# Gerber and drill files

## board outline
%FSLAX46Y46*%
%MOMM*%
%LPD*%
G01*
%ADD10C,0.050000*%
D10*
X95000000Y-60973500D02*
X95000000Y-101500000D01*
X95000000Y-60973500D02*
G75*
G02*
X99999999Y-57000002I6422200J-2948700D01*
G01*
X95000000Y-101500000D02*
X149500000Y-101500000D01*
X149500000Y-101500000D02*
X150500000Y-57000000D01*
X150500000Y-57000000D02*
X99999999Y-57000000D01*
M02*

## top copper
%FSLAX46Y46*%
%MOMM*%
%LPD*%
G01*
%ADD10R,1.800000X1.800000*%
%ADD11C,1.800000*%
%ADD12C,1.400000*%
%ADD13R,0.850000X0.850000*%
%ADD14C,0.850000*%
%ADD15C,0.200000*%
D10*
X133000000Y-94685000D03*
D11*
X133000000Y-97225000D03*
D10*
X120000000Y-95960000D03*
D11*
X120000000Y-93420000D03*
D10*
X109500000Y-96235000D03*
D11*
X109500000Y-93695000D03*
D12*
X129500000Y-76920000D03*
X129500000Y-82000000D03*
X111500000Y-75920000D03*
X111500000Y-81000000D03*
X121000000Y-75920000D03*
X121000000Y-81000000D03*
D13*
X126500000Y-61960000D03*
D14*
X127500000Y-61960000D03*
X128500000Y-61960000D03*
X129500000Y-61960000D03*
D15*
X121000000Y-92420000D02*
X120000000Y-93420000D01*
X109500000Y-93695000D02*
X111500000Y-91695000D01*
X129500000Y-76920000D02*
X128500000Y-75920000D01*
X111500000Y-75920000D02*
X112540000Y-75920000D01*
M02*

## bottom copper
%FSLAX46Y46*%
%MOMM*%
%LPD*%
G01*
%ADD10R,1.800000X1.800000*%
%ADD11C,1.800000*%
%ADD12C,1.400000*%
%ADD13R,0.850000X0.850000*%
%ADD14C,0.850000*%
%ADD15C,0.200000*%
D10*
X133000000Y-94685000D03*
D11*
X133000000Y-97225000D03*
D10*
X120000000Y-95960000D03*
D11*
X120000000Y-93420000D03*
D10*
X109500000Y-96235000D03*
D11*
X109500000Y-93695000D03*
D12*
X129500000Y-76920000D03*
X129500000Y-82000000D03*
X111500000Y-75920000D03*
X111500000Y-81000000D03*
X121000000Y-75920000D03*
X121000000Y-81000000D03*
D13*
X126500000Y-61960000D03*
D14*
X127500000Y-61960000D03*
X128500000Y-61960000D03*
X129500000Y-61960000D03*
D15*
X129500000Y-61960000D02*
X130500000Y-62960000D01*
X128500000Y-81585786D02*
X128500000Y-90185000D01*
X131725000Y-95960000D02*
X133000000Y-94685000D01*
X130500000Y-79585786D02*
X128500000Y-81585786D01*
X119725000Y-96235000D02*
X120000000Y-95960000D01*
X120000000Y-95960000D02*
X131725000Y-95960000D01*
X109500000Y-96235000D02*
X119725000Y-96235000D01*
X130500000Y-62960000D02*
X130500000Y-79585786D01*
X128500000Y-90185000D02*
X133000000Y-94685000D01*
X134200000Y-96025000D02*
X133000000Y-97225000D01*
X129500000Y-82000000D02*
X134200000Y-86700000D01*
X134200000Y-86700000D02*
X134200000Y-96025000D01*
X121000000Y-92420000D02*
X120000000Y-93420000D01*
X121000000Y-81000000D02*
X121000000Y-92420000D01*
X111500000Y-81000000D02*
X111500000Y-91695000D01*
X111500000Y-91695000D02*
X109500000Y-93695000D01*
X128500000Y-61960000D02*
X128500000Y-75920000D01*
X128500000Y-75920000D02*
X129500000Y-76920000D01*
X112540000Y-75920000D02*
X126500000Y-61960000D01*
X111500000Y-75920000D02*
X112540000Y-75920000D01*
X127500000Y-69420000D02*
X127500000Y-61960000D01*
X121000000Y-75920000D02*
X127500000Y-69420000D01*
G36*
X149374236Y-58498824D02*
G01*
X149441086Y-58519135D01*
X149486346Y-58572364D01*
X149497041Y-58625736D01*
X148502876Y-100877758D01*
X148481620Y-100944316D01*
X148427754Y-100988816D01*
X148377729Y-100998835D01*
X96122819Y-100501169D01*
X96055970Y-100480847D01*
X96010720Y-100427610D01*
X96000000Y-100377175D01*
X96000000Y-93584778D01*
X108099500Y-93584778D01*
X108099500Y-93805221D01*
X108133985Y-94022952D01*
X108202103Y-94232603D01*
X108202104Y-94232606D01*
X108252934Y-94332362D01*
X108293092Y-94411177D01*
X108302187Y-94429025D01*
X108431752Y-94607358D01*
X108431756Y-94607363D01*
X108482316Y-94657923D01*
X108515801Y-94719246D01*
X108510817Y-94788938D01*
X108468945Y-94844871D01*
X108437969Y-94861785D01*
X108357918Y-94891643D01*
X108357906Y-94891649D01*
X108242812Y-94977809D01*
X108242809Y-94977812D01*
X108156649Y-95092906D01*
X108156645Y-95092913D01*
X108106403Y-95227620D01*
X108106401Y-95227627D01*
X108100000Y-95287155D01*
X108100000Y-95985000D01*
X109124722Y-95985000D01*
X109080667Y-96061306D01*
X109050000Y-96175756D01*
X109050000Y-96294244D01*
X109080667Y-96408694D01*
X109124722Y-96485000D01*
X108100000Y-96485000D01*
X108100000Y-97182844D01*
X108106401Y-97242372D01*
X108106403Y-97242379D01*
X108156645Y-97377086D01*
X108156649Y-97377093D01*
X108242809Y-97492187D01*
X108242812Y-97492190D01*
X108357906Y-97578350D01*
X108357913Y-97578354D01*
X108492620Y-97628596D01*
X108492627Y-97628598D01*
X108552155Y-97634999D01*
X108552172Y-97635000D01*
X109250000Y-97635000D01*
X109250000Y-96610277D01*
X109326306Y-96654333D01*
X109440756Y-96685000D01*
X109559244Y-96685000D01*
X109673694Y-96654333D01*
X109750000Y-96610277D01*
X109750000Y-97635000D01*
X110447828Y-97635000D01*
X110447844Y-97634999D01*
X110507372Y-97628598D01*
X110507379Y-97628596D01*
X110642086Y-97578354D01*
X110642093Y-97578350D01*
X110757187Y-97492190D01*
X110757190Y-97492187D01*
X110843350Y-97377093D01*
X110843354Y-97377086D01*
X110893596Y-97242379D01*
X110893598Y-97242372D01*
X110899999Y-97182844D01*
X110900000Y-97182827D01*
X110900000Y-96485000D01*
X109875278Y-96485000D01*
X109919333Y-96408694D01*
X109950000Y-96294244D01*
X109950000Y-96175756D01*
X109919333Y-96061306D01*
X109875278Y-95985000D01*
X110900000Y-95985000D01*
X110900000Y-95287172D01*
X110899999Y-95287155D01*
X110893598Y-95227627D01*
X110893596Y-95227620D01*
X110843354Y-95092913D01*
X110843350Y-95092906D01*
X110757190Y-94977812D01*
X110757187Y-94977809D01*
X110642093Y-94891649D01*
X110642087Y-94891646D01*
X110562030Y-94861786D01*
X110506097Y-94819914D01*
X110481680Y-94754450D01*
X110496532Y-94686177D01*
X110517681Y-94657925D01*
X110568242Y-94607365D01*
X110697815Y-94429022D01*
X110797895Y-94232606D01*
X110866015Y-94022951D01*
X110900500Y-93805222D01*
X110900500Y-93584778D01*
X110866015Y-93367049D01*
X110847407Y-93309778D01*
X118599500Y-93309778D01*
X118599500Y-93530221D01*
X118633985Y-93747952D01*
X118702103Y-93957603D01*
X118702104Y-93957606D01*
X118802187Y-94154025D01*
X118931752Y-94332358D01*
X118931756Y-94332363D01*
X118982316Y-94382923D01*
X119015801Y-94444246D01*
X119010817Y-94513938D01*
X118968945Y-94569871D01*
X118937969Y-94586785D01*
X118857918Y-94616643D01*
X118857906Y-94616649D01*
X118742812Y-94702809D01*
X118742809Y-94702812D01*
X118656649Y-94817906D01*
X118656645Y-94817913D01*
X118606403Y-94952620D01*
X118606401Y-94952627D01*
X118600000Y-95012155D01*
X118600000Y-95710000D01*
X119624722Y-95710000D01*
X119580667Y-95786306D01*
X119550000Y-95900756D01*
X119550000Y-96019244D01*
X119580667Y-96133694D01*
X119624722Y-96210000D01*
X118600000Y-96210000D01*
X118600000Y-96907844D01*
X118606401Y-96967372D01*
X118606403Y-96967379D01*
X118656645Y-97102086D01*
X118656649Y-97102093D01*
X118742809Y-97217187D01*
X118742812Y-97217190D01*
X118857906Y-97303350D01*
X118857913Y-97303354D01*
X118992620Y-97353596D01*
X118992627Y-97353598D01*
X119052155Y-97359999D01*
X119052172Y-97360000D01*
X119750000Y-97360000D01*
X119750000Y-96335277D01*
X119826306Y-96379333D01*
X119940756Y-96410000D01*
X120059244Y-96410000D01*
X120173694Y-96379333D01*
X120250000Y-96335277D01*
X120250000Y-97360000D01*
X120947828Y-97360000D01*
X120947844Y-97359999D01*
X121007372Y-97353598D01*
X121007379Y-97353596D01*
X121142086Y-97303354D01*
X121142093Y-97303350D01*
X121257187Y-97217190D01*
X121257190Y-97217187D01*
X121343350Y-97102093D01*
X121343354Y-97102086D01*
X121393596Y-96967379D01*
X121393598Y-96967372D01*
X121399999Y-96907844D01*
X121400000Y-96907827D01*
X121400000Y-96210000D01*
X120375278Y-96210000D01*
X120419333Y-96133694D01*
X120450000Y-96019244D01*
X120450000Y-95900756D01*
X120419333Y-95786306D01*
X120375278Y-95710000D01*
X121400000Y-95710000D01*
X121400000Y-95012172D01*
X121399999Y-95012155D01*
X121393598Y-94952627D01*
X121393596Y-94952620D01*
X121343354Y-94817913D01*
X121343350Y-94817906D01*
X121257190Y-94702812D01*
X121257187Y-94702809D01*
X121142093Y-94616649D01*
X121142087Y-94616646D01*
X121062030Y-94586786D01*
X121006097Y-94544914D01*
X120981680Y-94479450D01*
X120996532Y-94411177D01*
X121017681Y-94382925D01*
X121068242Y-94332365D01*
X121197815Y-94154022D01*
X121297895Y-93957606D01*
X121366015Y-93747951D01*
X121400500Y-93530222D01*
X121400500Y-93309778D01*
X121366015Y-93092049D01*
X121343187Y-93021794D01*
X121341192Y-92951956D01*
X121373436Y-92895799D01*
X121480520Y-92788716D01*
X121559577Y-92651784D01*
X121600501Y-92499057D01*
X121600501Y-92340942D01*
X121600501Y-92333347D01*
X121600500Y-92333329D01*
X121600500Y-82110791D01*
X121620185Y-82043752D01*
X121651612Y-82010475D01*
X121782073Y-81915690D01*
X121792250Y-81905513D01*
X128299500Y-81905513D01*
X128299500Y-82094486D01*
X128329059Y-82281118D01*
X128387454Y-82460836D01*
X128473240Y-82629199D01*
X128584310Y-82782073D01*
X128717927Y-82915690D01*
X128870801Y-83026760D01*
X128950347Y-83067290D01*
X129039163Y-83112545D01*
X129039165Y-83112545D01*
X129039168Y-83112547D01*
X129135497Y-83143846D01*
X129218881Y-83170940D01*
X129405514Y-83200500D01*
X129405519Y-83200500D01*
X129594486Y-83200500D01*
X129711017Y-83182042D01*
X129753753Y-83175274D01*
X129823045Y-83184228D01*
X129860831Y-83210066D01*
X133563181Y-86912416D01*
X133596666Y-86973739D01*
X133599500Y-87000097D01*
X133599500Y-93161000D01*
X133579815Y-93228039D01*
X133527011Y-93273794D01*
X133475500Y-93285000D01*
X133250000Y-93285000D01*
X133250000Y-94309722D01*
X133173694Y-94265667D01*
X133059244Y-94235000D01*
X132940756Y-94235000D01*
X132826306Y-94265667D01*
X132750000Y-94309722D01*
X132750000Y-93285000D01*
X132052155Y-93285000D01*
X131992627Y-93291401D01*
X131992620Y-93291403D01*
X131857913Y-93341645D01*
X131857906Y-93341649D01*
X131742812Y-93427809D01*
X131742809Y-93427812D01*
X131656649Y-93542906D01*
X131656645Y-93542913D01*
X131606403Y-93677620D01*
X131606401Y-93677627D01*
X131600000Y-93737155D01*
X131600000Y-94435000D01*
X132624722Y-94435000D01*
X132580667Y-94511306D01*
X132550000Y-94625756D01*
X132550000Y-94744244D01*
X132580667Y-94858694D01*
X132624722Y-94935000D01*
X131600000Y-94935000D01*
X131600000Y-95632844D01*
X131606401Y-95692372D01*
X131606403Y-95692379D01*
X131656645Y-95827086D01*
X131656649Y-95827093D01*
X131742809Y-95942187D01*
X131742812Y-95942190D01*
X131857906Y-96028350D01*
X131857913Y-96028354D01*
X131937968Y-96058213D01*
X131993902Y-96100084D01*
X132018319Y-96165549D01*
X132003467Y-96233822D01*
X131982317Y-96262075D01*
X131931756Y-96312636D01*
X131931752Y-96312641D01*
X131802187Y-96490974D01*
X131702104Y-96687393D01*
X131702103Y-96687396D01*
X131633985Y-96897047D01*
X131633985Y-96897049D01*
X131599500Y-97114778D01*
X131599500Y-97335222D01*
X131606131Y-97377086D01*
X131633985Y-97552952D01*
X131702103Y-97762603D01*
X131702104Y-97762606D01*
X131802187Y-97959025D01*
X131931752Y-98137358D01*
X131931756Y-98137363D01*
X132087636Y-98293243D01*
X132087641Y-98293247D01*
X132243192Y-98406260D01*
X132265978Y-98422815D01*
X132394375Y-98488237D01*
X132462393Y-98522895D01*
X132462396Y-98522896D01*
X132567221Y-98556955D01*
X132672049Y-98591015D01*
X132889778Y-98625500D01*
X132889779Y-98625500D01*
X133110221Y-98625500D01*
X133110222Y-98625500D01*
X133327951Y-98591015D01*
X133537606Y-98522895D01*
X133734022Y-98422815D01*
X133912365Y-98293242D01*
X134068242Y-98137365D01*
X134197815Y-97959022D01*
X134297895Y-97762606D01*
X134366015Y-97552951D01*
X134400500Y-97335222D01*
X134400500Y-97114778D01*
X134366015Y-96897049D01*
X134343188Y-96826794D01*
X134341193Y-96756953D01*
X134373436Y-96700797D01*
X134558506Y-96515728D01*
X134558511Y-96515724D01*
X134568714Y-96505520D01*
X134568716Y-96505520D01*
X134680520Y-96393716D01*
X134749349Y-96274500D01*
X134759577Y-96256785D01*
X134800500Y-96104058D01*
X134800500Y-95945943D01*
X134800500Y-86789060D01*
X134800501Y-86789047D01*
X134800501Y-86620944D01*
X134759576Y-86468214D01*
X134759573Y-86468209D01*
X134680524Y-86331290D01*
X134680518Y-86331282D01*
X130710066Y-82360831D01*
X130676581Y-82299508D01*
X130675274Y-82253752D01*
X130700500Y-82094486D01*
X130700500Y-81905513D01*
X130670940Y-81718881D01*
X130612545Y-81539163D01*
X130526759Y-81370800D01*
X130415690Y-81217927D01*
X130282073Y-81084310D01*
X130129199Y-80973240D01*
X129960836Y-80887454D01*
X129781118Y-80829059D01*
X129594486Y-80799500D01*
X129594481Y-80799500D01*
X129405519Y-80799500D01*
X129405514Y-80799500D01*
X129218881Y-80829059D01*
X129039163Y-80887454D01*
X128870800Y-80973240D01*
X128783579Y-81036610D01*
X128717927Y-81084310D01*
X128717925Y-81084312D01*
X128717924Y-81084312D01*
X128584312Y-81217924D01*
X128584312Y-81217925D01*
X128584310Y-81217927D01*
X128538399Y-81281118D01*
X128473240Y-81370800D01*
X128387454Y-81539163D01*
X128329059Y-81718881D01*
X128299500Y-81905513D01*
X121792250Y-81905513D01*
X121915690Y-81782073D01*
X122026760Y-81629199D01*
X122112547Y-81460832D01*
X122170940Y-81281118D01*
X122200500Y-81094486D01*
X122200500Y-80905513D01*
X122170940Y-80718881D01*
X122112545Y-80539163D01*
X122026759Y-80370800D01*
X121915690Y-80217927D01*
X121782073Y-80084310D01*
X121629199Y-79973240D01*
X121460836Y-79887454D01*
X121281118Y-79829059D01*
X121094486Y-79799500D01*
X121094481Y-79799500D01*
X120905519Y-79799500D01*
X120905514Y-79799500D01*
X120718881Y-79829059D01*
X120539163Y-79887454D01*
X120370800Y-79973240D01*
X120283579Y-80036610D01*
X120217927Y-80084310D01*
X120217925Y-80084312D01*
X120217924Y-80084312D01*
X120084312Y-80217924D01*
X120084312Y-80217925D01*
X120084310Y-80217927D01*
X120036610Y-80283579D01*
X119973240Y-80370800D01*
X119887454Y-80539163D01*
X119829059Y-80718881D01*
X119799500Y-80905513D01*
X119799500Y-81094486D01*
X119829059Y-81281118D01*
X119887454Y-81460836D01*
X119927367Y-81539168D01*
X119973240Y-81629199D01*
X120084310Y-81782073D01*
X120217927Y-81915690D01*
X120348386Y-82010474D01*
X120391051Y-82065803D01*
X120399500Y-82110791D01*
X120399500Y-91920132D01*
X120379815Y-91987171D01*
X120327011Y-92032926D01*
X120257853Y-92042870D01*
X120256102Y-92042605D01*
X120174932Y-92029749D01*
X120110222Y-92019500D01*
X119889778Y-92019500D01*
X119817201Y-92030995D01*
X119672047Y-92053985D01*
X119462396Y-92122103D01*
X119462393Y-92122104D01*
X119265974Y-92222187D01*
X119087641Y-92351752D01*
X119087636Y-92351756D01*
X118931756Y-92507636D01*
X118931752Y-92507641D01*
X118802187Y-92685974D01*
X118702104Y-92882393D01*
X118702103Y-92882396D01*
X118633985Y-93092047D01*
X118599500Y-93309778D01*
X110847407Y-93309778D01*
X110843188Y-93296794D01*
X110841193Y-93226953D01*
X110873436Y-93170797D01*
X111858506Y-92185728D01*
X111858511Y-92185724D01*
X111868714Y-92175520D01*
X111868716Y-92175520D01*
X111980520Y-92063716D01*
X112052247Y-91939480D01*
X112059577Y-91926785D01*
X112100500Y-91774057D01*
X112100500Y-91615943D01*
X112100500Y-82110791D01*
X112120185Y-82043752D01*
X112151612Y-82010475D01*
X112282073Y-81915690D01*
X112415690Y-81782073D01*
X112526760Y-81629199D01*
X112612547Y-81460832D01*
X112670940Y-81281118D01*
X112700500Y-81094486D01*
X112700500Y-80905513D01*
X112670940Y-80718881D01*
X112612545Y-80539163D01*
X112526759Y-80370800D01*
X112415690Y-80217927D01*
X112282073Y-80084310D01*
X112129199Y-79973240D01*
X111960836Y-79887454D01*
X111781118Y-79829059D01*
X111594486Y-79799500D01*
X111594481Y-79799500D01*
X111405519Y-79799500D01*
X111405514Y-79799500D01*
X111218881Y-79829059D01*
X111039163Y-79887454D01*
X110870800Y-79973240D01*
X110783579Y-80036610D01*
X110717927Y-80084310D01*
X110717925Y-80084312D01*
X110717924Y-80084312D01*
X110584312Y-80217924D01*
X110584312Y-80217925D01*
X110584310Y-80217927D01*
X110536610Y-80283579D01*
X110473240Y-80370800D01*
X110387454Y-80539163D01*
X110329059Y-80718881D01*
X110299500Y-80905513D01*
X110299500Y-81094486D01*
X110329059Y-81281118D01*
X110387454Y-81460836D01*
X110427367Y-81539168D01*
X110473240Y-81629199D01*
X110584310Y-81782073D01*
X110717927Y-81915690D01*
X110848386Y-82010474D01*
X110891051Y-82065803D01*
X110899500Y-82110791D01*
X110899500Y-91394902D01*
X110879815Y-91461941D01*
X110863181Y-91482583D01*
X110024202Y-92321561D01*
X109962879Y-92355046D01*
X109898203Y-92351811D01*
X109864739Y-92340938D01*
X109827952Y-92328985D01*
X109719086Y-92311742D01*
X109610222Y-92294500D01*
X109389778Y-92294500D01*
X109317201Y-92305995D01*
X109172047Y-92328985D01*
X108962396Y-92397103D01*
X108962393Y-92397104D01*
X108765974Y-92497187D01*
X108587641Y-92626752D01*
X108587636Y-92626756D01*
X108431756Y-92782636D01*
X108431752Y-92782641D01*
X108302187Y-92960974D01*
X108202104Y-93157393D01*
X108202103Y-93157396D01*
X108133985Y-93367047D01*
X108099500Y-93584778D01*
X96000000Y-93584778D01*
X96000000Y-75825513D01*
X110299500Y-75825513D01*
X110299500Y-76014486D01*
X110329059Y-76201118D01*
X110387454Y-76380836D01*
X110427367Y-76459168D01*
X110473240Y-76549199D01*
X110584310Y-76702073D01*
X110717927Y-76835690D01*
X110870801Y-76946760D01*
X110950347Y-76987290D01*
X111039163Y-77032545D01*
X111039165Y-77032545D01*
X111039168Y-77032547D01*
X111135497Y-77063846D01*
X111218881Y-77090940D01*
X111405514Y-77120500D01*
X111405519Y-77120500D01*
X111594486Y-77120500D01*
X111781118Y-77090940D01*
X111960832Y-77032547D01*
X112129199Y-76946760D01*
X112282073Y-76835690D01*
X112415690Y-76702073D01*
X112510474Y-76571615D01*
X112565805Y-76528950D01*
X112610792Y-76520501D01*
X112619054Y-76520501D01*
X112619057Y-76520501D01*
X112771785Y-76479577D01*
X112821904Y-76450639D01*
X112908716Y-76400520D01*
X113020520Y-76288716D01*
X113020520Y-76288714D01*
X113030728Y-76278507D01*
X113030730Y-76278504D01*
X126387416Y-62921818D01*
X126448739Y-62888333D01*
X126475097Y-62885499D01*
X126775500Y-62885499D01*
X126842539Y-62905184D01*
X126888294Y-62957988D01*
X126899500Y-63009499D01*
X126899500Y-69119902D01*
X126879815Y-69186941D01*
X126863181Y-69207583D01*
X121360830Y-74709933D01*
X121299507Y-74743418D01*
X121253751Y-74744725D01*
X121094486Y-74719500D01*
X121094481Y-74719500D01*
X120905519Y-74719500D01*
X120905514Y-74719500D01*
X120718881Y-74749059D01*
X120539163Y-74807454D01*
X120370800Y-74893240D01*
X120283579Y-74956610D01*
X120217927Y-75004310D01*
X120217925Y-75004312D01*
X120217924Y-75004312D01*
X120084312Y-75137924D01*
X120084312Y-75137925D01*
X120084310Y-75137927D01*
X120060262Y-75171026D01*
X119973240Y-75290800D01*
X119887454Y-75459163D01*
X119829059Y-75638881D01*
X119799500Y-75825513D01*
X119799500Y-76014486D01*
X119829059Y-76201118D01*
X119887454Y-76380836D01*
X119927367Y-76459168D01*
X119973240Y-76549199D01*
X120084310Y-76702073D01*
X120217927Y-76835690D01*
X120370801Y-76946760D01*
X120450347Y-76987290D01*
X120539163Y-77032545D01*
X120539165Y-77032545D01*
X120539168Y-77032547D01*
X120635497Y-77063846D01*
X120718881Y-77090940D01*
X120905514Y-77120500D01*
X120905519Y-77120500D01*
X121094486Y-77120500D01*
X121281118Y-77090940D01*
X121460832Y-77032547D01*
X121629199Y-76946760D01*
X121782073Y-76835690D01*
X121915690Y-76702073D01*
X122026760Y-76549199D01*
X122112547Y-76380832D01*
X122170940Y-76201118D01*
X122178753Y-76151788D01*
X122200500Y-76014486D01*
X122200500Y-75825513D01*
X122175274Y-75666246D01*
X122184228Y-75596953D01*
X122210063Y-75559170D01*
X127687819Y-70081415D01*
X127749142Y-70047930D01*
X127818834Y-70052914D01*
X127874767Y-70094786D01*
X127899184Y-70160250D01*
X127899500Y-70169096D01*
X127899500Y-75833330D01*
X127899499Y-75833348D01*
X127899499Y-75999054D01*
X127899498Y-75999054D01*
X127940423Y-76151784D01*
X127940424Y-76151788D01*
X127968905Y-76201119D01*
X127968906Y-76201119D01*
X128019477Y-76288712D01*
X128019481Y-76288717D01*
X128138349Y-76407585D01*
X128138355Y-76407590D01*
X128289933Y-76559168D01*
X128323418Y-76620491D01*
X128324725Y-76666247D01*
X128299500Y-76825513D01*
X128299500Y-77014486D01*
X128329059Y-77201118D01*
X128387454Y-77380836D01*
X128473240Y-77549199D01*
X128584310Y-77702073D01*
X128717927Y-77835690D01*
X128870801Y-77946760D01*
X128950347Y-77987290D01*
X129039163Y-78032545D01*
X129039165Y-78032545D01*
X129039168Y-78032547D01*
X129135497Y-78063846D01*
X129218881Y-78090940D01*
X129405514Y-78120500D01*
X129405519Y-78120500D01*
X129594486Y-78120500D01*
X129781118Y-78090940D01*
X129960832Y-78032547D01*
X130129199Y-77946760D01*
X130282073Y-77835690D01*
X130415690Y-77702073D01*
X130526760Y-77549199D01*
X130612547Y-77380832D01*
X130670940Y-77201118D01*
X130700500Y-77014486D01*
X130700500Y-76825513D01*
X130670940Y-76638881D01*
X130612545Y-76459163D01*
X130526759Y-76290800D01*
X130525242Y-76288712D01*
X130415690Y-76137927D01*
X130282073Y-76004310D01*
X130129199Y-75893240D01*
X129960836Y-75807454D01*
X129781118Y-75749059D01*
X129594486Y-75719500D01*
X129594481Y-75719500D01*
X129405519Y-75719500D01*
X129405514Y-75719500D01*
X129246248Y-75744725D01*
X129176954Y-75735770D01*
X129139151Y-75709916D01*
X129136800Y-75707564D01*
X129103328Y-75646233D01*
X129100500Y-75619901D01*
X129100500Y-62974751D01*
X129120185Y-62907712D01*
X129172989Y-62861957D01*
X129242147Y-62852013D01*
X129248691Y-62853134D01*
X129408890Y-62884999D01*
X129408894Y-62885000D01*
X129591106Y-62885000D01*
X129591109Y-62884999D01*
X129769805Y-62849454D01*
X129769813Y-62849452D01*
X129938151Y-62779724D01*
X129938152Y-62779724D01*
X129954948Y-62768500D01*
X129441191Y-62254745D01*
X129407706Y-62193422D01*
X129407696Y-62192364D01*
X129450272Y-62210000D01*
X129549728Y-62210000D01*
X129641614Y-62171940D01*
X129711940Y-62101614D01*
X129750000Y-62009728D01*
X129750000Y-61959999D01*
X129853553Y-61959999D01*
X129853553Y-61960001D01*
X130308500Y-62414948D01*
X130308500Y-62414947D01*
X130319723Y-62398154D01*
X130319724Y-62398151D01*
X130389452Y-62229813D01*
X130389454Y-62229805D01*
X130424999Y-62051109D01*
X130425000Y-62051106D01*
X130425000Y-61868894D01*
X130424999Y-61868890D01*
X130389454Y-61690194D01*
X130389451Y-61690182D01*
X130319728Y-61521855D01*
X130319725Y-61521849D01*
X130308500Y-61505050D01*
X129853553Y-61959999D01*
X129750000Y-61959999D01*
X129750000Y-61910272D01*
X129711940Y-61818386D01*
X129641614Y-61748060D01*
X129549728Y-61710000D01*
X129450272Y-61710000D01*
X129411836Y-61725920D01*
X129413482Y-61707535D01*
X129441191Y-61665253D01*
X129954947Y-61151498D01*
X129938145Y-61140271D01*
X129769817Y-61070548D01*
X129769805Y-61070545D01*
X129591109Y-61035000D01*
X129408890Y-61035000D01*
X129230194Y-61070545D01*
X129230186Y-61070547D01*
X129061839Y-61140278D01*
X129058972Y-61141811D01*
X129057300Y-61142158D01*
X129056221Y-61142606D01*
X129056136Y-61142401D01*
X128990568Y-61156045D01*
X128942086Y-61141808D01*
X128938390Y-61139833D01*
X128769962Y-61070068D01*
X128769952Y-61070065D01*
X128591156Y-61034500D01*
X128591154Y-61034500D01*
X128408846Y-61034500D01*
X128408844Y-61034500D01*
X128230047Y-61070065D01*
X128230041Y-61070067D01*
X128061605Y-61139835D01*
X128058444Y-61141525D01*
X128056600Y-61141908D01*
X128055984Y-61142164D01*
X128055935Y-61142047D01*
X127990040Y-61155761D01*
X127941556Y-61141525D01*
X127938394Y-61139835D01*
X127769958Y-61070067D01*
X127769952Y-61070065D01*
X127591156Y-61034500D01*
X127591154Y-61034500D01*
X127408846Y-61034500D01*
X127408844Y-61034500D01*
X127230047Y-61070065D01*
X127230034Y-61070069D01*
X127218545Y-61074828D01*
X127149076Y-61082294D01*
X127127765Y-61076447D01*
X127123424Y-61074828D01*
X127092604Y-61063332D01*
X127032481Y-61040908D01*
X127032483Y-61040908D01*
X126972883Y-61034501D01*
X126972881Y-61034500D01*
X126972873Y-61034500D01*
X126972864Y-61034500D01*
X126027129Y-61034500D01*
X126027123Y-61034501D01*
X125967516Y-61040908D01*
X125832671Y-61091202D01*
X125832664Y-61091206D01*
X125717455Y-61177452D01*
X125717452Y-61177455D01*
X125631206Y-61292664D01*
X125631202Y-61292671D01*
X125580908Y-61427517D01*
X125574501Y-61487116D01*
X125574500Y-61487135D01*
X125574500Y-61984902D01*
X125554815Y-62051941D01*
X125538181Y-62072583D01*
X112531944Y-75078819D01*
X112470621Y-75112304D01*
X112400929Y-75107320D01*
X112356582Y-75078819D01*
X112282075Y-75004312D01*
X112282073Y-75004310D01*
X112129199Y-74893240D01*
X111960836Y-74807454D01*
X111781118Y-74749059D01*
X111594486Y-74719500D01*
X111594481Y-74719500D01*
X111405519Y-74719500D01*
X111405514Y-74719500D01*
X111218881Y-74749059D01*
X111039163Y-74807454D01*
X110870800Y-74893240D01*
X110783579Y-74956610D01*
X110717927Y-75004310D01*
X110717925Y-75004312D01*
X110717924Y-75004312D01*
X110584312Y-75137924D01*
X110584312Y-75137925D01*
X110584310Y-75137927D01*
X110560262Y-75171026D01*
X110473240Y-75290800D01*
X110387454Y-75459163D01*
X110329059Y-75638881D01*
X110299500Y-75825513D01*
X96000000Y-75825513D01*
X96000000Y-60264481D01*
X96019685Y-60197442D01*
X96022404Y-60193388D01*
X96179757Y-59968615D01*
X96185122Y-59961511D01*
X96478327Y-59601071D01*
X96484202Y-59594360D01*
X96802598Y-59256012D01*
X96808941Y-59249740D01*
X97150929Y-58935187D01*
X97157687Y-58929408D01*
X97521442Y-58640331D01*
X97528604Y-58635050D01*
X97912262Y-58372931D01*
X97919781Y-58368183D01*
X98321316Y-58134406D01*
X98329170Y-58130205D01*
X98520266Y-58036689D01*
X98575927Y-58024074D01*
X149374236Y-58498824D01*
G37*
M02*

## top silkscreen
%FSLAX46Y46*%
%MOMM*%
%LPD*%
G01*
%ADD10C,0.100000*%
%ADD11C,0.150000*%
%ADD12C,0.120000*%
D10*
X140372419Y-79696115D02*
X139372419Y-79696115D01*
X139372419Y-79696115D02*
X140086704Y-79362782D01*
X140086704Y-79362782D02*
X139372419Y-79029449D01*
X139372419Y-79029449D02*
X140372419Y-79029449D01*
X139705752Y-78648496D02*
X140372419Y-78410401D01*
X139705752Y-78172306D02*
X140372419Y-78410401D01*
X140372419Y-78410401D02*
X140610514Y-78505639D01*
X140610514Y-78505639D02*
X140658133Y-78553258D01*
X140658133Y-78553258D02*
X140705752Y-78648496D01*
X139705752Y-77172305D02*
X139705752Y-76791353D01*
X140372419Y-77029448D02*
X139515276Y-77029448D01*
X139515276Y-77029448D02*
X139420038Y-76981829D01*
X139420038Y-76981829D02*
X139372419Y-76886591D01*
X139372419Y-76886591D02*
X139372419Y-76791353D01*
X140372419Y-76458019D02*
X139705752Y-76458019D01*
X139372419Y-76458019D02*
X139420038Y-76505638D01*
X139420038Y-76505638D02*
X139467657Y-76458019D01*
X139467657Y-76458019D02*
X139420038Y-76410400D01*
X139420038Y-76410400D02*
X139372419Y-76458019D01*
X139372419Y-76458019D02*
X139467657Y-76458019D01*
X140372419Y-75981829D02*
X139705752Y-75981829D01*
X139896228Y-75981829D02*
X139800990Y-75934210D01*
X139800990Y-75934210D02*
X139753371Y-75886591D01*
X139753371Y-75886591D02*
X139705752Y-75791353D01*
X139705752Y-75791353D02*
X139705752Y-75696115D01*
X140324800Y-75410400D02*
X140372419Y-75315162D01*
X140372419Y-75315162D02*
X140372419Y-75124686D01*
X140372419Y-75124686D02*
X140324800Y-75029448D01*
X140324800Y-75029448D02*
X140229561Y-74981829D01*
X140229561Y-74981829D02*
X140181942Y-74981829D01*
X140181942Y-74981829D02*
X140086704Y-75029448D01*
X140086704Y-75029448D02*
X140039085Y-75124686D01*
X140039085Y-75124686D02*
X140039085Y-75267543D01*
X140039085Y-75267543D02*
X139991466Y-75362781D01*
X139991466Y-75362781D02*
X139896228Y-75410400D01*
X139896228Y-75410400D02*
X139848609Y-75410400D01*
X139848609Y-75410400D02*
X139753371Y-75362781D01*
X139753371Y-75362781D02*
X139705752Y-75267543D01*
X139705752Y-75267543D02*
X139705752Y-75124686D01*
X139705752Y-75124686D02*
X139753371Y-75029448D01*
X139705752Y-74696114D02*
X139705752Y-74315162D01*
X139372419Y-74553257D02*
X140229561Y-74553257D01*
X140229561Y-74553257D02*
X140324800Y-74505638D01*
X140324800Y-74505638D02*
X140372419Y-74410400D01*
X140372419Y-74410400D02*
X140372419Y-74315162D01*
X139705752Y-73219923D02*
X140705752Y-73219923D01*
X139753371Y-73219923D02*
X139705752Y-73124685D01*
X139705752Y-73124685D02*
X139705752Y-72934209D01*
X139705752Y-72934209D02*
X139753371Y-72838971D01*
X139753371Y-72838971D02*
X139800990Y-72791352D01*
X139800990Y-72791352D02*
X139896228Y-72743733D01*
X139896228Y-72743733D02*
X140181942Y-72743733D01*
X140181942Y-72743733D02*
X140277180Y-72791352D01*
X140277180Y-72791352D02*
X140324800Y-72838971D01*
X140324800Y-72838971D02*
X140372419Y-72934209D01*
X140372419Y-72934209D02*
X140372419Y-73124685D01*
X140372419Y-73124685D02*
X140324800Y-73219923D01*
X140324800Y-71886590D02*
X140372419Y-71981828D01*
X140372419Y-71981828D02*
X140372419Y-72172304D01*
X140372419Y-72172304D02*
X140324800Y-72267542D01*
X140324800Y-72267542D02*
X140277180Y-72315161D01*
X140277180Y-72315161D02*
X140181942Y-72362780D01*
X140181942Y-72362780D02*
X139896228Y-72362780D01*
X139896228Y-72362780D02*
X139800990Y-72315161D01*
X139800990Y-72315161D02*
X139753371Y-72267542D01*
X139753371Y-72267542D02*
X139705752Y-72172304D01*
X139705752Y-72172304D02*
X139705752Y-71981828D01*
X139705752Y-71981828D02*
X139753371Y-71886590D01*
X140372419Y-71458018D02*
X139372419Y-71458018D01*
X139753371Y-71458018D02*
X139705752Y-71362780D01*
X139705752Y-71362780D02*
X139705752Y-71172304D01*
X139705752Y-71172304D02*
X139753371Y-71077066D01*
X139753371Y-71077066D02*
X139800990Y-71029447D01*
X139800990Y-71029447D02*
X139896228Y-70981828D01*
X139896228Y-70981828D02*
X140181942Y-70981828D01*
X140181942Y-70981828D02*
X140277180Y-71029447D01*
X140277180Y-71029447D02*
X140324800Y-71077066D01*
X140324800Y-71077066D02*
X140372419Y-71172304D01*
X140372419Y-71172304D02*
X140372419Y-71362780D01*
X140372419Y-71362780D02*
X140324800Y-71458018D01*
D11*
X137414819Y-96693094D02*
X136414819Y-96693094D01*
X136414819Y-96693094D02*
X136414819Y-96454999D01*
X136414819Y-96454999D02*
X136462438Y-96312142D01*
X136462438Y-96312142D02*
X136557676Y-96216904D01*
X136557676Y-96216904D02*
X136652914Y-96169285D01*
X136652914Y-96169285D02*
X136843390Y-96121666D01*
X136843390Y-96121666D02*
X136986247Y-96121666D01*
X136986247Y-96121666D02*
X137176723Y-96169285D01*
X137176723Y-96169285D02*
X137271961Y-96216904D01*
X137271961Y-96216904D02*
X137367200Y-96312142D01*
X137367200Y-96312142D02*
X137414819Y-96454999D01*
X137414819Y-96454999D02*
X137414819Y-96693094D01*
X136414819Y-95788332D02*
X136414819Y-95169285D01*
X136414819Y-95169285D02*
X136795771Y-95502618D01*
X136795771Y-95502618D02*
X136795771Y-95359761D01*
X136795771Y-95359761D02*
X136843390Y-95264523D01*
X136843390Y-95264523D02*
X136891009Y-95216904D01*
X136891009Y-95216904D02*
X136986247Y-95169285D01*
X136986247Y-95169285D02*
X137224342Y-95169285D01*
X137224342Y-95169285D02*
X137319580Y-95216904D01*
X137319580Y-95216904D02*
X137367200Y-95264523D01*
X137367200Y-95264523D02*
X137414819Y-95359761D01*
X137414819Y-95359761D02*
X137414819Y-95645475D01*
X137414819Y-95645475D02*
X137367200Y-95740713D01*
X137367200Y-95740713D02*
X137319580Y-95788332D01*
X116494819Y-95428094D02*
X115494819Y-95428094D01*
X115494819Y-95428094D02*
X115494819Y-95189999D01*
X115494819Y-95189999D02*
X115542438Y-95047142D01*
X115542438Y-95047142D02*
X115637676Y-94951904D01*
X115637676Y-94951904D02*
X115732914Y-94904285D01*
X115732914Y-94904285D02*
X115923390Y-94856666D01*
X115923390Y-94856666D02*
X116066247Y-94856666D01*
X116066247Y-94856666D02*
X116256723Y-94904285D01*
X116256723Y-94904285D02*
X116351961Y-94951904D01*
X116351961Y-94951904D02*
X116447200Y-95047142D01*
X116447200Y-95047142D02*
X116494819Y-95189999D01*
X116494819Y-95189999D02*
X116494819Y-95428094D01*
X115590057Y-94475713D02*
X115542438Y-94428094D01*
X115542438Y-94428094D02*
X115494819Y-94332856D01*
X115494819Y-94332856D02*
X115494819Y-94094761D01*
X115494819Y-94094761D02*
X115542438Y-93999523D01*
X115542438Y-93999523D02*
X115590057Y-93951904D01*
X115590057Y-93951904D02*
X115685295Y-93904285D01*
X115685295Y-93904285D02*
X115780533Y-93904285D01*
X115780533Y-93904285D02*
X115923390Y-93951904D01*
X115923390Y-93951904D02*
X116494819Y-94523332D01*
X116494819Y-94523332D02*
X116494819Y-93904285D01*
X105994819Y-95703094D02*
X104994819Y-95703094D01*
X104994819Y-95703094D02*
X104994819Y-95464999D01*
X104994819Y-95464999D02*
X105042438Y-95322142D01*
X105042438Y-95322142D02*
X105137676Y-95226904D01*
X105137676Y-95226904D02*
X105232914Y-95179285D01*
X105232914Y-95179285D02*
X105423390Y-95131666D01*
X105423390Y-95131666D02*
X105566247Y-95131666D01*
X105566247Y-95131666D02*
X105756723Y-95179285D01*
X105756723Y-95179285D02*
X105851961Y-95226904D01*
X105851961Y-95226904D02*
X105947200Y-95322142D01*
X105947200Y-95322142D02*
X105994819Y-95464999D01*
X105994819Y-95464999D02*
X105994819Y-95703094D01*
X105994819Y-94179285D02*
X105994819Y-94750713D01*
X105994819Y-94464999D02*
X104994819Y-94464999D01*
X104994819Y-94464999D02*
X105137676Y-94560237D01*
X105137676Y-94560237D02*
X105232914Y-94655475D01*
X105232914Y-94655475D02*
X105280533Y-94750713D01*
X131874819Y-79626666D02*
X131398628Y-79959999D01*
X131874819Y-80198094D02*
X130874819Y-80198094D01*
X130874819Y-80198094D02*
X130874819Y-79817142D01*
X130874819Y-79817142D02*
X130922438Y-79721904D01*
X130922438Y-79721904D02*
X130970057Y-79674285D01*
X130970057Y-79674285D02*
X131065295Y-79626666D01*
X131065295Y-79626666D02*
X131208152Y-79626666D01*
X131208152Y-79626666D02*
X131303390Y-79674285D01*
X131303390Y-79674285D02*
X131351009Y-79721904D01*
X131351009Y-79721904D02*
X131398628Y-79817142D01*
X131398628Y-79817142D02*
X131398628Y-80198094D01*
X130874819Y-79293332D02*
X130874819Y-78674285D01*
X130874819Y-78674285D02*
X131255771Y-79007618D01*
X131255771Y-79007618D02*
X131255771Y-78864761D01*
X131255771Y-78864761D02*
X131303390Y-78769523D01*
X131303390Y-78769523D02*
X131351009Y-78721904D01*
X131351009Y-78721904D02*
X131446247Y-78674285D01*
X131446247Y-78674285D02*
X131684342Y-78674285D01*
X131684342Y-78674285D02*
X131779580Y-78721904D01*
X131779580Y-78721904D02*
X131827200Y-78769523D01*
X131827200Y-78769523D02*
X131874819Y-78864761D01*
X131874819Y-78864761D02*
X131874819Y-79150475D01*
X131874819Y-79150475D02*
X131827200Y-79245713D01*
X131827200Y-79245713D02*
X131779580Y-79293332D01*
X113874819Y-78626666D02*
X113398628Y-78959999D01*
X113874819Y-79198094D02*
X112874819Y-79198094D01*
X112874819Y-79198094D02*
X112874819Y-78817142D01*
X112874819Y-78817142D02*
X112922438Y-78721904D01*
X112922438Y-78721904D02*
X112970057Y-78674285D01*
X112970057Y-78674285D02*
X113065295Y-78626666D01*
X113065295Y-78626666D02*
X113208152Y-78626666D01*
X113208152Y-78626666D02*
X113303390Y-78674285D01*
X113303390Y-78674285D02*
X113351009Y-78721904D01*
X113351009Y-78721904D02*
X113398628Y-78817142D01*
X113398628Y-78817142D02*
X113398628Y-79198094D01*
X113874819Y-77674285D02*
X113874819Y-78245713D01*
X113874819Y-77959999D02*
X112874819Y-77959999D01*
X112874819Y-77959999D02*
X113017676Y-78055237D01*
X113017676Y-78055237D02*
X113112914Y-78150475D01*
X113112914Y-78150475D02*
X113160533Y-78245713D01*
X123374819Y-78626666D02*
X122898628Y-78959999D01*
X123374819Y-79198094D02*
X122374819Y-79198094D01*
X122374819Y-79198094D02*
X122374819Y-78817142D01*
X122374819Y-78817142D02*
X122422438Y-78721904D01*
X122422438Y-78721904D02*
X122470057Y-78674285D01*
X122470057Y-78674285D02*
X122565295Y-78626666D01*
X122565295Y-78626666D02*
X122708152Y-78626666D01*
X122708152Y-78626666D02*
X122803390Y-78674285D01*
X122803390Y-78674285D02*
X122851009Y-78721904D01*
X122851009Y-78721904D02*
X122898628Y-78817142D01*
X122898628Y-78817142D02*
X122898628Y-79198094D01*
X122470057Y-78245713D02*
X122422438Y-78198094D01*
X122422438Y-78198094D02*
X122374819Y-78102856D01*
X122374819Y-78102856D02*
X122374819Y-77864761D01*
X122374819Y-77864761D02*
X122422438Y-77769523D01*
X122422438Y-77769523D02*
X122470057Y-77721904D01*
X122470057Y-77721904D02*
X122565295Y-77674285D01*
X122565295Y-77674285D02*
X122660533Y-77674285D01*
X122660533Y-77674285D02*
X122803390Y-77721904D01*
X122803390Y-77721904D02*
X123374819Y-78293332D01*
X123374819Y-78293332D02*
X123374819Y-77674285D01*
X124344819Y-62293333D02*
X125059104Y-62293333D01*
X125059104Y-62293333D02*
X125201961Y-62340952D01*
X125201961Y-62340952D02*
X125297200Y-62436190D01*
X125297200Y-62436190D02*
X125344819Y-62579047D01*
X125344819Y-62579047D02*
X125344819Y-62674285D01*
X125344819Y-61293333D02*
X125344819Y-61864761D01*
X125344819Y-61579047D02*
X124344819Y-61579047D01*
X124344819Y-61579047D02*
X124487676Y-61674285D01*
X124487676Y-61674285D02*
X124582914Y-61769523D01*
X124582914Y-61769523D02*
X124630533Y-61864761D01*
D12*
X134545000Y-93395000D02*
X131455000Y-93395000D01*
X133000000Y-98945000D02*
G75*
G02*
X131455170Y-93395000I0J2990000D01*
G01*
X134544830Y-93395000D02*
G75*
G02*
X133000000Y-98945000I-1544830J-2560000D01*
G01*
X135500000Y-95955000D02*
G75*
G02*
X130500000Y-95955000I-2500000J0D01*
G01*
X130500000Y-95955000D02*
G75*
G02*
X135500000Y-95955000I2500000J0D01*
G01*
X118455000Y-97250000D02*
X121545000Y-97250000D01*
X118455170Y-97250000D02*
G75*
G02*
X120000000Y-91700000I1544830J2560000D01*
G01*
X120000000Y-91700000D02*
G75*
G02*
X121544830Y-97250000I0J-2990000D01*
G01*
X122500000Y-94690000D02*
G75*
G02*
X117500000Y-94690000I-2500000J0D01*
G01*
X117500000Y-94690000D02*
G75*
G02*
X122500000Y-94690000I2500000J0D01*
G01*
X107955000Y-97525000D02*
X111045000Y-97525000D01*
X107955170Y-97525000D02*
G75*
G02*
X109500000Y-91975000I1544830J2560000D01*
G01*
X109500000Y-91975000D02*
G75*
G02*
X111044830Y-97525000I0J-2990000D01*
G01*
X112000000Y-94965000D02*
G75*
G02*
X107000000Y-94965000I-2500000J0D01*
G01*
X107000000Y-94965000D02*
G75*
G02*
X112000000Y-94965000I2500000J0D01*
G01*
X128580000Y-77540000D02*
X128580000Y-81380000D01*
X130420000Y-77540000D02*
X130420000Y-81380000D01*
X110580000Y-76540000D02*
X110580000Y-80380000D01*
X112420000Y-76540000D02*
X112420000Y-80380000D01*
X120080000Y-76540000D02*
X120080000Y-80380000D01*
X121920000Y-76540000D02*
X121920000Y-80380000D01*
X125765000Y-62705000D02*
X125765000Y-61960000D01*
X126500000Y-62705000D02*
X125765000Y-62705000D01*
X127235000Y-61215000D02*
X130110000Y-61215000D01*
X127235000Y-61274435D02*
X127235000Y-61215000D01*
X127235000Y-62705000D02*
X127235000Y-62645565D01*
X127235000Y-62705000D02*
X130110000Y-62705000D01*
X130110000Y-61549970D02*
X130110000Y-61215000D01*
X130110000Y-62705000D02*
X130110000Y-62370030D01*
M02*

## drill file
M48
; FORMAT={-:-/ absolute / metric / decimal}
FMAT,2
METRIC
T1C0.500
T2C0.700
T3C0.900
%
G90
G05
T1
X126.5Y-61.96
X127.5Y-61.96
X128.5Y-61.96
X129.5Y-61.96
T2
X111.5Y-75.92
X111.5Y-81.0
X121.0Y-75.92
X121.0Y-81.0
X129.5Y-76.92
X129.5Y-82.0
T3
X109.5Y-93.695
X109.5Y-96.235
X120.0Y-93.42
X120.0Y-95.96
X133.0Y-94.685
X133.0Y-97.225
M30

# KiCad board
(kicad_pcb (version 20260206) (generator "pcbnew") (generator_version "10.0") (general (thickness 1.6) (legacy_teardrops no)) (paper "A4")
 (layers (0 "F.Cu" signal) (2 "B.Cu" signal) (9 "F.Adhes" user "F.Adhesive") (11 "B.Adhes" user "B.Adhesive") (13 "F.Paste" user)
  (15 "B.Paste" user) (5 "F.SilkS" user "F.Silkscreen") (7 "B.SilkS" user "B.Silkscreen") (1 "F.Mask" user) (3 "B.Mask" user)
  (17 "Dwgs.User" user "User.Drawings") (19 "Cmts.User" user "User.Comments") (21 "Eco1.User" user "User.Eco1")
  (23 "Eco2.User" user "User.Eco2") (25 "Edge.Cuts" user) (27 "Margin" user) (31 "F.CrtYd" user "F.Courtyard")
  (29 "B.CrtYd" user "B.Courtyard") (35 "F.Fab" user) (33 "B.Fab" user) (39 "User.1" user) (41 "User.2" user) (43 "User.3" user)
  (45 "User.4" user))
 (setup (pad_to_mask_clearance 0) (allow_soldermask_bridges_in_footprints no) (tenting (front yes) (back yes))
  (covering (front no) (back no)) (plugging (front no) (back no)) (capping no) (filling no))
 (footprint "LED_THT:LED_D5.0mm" (layer "F.Cu") (at 133 94.685 -90)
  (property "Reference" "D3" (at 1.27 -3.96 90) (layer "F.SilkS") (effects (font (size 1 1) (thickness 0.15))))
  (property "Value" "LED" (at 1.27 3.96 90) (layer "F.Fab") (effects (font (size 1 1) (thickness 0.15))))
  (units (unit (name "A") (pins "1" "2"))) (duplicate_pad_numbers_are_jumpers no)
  (fp_line (start -1.29 -1.545) (end -1.29 1.545) (stroke (width 0.12) (type solid)) (layer "F.SilkS"))
  (fp_arc (start 4.26 0) (mid 2.071779 2.880495) (end -1.29 1.54483) (stroke (width 0.12) (type solid)) (layer "F.SilkS"))
  (fp_arc (start -1.29 -1.54483) (mid 2.071779 -2.880495) (end 4.26 0) (stroke (width 0.12) (type solid)) (layer "F.SilkS"))
  (fp_circle (center 1.27 0) (end 3.77 0) (stroke (width 0.12) (type solid)) (fill no) (layer "F.SilkS"))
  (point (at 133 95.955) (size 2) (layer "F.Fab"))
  (pad "1" thru_hole rect (at 0 0 270) (size 1.8 1.8) (drill 0.9) (layers "*.Cu" "*.Mask") (remove_unused_layers no) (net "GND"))
  (pad "2" thru_hole circle (at 2.54 0 270) (size 1.8 1.8) (drill 0.9) (layers "*.Cu" "*.Mask") (remove_unused_layers no) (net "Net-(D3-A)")))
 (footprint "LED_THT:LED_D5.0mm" (layer "F.Cu") (at 120 95.96 90)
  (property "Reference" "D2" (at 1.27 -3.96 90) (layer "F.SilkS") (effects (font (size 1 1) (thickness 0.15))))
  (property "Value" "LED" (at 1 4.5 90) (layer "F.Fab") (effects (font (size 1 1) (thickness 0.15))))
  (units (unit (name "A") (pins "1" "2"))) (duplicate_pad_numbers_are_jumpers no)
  (fp_line (start -1.29 -1.545) (end -1.29 1.545) (stroke (width 0.12) (type solid)) (layer "F.SilkS"))
  (fp_arc (start -1.29 -1.54483) (mid 2.071779 -2.880495) (end 4.26 0) (stroke (width 0.12) (type solid)) (layer "F.SilkS"))
  (fp_arc (start 4.26 0) (mid 2.071779 2.880495) (end -1.29 1.54483) (stroke (width 0.12) (type solid)) (layer "F.SilkS"))
  (fp_circle (center 1.27 0) (end 3.77 0) (stroke (width 0.12) (type solid)) (fill no) (layer "F.SilkS"))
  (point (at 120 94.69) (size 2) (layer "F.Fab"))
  (pad "1" thru_hole rect (at 0 0 90) (size 1.8 1.8) (drill 0.9) (layers "*.Cu" "*.Mask") (remove_unused_layers no) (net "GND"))
  (pad "2" thru_hole circle (at 2.54 0 90) (size 1.8 1.8) (drill 0.9) (layers "*.Cu" "*.Mask") (remove_unused_layers no) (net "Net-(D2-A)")))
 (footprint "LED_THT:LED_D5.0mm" (layer "F.Cu") (at 109.5 96.235 90)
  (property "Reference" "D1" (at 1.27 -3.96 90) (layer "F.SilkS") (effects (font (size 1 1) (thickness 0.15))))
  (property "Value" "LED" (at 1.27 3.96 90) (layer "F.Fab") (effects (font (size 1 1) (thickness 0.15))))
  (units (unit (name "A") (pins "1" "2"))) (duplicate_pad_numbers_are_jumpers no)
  (fp_line (start -1.29 -1.545) (end -1.29 1.545) (stroke (width 0.12) (type solid)) (layer "F.SilkS"))
  (fp_arc (start -1.29 -1.54483) (mid 2.071779 -2.880495) (end 4.26 0) (stroke (width 0.12) (type solid)) (layer "F.SilkS"))
  (fp_arc (start 4.26 0) (mid 2.071779 2.880495) (end -1.29 1.54483) (stroke (width 0.12) (type solid)) (layer "F.SilkS"))
  (fp_circle (center 1.27 0) (end 3.77 0) (stroke (width 0.12) (type solid)) (fill no) (layer "F.SilkS"))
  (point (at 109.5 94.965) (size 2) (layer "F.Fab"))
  (pad "1" thru_hole rect (at 0 0 90) (size 1.8 1.8) (drill 0.9) (layers "*.Cu" "*.Mask") (remove_unused_layers no) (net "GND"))
  (pad "2" thru_hole circle (at 2.54 0 90) (size 1.8 1.8) (drill 0.9) (layers "*.Cu" "*.Mask") (remove_unused_layers no) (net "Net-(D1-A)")))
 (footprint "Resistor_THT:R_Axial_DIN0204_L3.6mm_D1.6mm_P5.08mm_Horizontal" (layer "F.Cu") (at 129.5 76.92 -90)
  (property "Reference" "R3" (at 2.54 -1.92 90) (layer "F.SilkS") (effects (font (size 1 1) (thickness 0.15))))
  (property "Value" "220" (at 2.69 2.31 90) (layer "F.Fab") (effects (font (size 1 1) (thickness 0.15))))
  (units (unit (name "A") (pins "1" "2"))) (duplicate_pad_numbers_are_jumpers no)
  (fp_line (start 0.62 0.92) (end 4.46 0.92) (stroke (width 0.12) (type solid)) (layer "F.SilkS"))
  (fp_line (start 0.62 -0.92) (end 4.46 -0.92) (stroke (width 0.12) (type solid)) (layer "F.SilkS"))
  (pad "1" thru_hole circle (at 0 0 270) (size 1.4 1.4) (drill 0.7) (layers "*.Cu" "*.Mask") (remove_unused_layers no)
   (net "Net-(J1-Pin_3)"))
  (pad "2" thru_hole circle (at 5.08 0 270) (size 1.4 1.4) (drill 0.7) (layers "*.Cu" "*.Mask") (remove_unused_layers no) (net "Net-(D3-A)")))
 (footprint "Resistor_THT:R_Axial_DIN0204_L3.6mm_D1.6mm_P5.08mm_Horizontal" (layer "F.Cu") (at 111.5 75.92 -90)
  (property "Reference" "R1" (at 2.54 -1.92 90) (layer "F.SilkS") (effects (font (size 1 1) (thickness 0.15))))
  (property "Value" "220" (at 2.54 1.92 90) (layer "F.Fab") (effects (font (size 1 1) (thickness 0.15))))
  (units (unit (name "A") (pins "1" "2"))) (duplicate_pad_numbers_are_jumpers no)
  (fp_line (start 0.62 0.92) (end 4.46 0.92) (stroke (width 0.12) (type solid)) (layer "F.SilkS"))
  (fp_line (start 0.62 -0.92) (end 4.46 -0.92) (stroke (width 0.12) (type solid)) (layer "F.SilkS"))
  (pad "1" thru_hole circle (at 0 0 270) (size 1.4 1.4) (drill 0.7) (layers "*.Cu" "*.Mask") (remove_unused_layers no)
   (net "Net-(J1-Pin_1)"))
  (pad "2" thru_hole circle (at 5.08 0 270) (size 1.4 1.4) (drill 0.7) (layers "*.Cu" "*.Mask") (remove_unused_layers no) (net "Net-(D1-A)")))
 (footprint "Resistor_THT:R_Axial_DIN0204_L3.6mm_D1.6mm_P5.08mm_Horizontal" (layer "F.Cu") (at 121 75.92 -90)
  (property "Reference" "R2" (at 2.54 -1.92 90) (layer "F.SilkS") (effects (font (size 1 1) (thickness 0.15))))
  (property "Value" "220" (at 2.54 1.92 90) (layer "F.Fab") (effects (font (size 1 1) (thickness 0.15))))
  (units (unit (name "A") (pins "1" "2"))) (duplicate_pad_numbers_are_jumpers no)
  (fp_line (start 0.62 0.92) (end 4.46 0.92) (stroke (width 0.12) (type solid)) (layer "F.SilkS"))
  (fp_line (start 0.62 -0.92) (end 4.46 -0.92) (stroke (width 0.12) (type solid)) (layer "F.SilkS"))
  (pad "1" thru_hole circle (at 0 0 270) (size 1.4 1.4) (drill 0.7) (layers "*.Cu" "*.Mask") (remove_unused_layers no)
   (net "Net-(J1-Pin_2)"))
  (pad "2" thru_hole circle (at 5.08 0 270) (size 1.4 1.4) (drill 0.7) (layers "*.Cu" "*.Mask") (remove_unused_layers no) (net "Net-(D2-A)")))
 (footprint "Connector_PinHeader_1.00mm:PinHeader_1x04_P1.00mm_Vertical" (layer "F.Cu") (at 126.5 61.96 90)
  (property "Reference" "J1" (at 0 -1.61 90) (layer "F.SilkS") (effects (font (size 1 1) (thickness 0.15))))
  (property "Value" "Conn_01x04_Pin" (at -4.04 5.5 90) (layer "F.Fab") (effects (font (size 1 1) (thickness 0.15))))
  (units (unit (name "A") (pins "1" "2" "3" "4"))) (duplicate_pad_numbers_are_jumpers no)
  (fp_line (start -0.745 -0.735) (end 0 -0.735) (stroke (width 0.12) (type solid)) (layer "F.SilkS"))
  (fp_line (start -0.745 0) (end -0.745 -0.735) (stroke (width 0.12) (type solid)) (layer "F.SilkS"))
  (fp_line (start 0.745 0.735) (end 0.745 3.61) (stroke (width 0.12) (type solid)) (layer "F.SilkS"))
  (fp_line (start 0.685565 0.735) (end 0.745 0.735) (stroke (width 0.12) (type solid)) (layer "F.SilkS"))
  (fp_line (start -0.745 0.735) (end -0.685565 0.735) (stroke (width 0.12) (type solid)) (layer "F.SilkS"))
  (fp_line (start -0.745 0.735) (end -0.745 3.61) (stroke (width 0.12) (type solid)) (layer "F.SilkS"))
  (fp_line (start 0.41003 3.61) (end 0.745 3.61) (stroke (width 0.12) (type solid)) (layer "F.SilkS"))
  (fp_line (start -0.745 3.61) (end -0.41003 3.61) (stroke (width 0.12) (type solid)) (layer "F.SilkS"))
  (pad "1" thru_hole rect (at 0 0 90) (size 0.85 0.85) (drill 0.5) (layers "*.Cu" "*.Mask") (remove_unused_layers no) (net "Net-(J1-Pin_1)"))
  (pad "2" thru_hole circle (at 0 1 90) (size 0.85 0.85) (drill 0.5) (layers "*.Cu" "*.Mask") (remove_unused_layers no)
   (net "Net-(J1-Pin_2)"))
  (pad "3" thru_hole circle (at 0 2 90) (size 0.85 0.85) (drill 0.5) (layers "*.Cu" "*.Mask") (remove_unused_layers no)
   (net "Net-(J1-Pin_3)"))
  (pad "4" thru_hole circle (at 0 3 90) (size 0.85 0.85) (drill 0.5) (layers "*.Cu" "*.Mask") (remove_unused_layers no) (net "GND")))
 (gr_line (start 95 60.9735) (end 95 101.5) (stroke (width 0.05) (type default)) (layer "Edge.Cuts"))
 (gr_arc (start 95 60.9735) (mid 97.025517 58.389691) (end 99.999999 57) (stroke (width 0.05) (type default)) (layer "Edge.Cuts"))
 (gr_line (start 95 101.5) (end 149.5 101.5) (stroke (width 0.05) (type default)) (layer "Edge.Cuts"))
 (gr_line (start 149.5 101.5) (end 150.5 57) (stroke (width 0.05) (type default)) (layer "Edge.Cuts"))
 (gr_line (start 150.5 57) (end 99.999999 57) (stroke (width 0.05) (type default)) (layer "Edge.Cuts"))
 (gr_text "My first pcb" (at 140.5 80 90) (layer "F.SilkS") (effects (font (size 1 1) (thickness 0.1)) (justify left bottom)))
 (segment (start 129.5 61.96) (end 130.5 62.96) (width 0.2) (layer "B.Cu") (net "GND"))
 (segment (start 128.5 81.585786) (end 128.5 90.185) (width 0.2) (layer "B.Cu") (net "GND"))
 (segment (start 131.725 95.96) (end 133 94.685) (width 0.2) (layer "B.Cu") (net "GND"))
 (segment (start 130.5 79.585786) (end 128.5 81.585786) (width 0.2) (layer "B.Cu") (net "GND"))
 (segment (start 119.725 96.235) (end 120 95.96) (width 0.2) (layer "B.Cu") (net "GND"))
 (segment (start 120 95.96) (end 131.725 95.96) (width 0.2) (layer "B.Cu") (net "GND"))
 (segment (start 109.5 96.235) (end 119.725 96.235) (width 0.2) (layer "B.Cu") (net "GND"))
 (segment (start 130.5 62.96) (end 130.5 79.585786) (width 0.2) (layer "B.Cu") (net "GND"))
 (segment (start 128.5 90.185) (end 133 94.685) (width 0.2) (layer "B.Cu") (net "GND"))
 (segment (start 134.2 96.025) (end 133 97.225) (width 0.2) (layer "B.Cu") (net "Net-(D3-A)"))
 (segment (start 129.5 82) (end 134.2 86.7) (width 0.2) (layer "B.Cu") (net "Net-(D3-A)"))
 (segment (start 134.2 86.7) (end 134.2 96.025) (width 0.2) (layer "B.Cu") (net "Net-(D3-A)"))
 (segment (start 121 92.42) (end 120 93.42) (width 0.2) (layer "F.Cu") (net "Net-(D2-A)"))
 (segment (start 121 92.42) (end 120 93.42) (width 0.2) (layer "B.Cu") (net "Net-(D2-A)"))
 (segment (start 121 81) (end 121 92.42) (width 0.2) (layer "B.Cu") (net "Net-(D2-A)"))
 (segment (start 109.5 93.695) (end 111.5 91.695) (width 0.2) (layer "F.Cu") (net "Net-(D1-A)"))
 (segment (start 111.5 81) (end 111.5 91.695) (width 0.2) (layer "B.Cu") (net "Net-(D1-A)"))
 (segment (start 111.5 91.695) (end 109.5 93.695) (width 0.2) (layer "B.Cu") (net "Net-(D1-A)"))
 (segment (start 129.5 76.92) (end 128.5 75.92) (width 0.2) (layer "F.Cu") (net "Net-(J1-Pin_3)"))
 (segment (start 128.5 61.96) (end 128.5 75.92) (width 0.2) (layer "B.Cu") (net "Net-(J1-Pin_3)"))
 (segment (start 128.5 75.92) (end 129.5 76.92) (width 0.2) (layer "B.Cu") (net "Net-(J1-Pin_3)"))
 (segment (start 111.5 75.92) (end 112.54 75.92) (width 0.2) (layer "F.Cu") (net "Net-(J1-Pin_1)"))
 (segment (start 112.54 75.92) (end 126.5 61.96) (width 0.2) (layer "B.Cu") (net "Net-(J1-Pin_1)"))
 (segment (start 111.5 75.92) (end 112.54 75.92) (width 0.2) (layer "B.Cu") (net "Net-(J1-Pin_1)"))
 (segment (start 127.5 69.42) (end 127.5 61.96) (width 0.2) (layer "B.Cu") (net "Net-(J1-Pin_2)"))
 (segment (start 121 75.92) (end 127.5 69.42) (width 0.2) (layer "B.Cu") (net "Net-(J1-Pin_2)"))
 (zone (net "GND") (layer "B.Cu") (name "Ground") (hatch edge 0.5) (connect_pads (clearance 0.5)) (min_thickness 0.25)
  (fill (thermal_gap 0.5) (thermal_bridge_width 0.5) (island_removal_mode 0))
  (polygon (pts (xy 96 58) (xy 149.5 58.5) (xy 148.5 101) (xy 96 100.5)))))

